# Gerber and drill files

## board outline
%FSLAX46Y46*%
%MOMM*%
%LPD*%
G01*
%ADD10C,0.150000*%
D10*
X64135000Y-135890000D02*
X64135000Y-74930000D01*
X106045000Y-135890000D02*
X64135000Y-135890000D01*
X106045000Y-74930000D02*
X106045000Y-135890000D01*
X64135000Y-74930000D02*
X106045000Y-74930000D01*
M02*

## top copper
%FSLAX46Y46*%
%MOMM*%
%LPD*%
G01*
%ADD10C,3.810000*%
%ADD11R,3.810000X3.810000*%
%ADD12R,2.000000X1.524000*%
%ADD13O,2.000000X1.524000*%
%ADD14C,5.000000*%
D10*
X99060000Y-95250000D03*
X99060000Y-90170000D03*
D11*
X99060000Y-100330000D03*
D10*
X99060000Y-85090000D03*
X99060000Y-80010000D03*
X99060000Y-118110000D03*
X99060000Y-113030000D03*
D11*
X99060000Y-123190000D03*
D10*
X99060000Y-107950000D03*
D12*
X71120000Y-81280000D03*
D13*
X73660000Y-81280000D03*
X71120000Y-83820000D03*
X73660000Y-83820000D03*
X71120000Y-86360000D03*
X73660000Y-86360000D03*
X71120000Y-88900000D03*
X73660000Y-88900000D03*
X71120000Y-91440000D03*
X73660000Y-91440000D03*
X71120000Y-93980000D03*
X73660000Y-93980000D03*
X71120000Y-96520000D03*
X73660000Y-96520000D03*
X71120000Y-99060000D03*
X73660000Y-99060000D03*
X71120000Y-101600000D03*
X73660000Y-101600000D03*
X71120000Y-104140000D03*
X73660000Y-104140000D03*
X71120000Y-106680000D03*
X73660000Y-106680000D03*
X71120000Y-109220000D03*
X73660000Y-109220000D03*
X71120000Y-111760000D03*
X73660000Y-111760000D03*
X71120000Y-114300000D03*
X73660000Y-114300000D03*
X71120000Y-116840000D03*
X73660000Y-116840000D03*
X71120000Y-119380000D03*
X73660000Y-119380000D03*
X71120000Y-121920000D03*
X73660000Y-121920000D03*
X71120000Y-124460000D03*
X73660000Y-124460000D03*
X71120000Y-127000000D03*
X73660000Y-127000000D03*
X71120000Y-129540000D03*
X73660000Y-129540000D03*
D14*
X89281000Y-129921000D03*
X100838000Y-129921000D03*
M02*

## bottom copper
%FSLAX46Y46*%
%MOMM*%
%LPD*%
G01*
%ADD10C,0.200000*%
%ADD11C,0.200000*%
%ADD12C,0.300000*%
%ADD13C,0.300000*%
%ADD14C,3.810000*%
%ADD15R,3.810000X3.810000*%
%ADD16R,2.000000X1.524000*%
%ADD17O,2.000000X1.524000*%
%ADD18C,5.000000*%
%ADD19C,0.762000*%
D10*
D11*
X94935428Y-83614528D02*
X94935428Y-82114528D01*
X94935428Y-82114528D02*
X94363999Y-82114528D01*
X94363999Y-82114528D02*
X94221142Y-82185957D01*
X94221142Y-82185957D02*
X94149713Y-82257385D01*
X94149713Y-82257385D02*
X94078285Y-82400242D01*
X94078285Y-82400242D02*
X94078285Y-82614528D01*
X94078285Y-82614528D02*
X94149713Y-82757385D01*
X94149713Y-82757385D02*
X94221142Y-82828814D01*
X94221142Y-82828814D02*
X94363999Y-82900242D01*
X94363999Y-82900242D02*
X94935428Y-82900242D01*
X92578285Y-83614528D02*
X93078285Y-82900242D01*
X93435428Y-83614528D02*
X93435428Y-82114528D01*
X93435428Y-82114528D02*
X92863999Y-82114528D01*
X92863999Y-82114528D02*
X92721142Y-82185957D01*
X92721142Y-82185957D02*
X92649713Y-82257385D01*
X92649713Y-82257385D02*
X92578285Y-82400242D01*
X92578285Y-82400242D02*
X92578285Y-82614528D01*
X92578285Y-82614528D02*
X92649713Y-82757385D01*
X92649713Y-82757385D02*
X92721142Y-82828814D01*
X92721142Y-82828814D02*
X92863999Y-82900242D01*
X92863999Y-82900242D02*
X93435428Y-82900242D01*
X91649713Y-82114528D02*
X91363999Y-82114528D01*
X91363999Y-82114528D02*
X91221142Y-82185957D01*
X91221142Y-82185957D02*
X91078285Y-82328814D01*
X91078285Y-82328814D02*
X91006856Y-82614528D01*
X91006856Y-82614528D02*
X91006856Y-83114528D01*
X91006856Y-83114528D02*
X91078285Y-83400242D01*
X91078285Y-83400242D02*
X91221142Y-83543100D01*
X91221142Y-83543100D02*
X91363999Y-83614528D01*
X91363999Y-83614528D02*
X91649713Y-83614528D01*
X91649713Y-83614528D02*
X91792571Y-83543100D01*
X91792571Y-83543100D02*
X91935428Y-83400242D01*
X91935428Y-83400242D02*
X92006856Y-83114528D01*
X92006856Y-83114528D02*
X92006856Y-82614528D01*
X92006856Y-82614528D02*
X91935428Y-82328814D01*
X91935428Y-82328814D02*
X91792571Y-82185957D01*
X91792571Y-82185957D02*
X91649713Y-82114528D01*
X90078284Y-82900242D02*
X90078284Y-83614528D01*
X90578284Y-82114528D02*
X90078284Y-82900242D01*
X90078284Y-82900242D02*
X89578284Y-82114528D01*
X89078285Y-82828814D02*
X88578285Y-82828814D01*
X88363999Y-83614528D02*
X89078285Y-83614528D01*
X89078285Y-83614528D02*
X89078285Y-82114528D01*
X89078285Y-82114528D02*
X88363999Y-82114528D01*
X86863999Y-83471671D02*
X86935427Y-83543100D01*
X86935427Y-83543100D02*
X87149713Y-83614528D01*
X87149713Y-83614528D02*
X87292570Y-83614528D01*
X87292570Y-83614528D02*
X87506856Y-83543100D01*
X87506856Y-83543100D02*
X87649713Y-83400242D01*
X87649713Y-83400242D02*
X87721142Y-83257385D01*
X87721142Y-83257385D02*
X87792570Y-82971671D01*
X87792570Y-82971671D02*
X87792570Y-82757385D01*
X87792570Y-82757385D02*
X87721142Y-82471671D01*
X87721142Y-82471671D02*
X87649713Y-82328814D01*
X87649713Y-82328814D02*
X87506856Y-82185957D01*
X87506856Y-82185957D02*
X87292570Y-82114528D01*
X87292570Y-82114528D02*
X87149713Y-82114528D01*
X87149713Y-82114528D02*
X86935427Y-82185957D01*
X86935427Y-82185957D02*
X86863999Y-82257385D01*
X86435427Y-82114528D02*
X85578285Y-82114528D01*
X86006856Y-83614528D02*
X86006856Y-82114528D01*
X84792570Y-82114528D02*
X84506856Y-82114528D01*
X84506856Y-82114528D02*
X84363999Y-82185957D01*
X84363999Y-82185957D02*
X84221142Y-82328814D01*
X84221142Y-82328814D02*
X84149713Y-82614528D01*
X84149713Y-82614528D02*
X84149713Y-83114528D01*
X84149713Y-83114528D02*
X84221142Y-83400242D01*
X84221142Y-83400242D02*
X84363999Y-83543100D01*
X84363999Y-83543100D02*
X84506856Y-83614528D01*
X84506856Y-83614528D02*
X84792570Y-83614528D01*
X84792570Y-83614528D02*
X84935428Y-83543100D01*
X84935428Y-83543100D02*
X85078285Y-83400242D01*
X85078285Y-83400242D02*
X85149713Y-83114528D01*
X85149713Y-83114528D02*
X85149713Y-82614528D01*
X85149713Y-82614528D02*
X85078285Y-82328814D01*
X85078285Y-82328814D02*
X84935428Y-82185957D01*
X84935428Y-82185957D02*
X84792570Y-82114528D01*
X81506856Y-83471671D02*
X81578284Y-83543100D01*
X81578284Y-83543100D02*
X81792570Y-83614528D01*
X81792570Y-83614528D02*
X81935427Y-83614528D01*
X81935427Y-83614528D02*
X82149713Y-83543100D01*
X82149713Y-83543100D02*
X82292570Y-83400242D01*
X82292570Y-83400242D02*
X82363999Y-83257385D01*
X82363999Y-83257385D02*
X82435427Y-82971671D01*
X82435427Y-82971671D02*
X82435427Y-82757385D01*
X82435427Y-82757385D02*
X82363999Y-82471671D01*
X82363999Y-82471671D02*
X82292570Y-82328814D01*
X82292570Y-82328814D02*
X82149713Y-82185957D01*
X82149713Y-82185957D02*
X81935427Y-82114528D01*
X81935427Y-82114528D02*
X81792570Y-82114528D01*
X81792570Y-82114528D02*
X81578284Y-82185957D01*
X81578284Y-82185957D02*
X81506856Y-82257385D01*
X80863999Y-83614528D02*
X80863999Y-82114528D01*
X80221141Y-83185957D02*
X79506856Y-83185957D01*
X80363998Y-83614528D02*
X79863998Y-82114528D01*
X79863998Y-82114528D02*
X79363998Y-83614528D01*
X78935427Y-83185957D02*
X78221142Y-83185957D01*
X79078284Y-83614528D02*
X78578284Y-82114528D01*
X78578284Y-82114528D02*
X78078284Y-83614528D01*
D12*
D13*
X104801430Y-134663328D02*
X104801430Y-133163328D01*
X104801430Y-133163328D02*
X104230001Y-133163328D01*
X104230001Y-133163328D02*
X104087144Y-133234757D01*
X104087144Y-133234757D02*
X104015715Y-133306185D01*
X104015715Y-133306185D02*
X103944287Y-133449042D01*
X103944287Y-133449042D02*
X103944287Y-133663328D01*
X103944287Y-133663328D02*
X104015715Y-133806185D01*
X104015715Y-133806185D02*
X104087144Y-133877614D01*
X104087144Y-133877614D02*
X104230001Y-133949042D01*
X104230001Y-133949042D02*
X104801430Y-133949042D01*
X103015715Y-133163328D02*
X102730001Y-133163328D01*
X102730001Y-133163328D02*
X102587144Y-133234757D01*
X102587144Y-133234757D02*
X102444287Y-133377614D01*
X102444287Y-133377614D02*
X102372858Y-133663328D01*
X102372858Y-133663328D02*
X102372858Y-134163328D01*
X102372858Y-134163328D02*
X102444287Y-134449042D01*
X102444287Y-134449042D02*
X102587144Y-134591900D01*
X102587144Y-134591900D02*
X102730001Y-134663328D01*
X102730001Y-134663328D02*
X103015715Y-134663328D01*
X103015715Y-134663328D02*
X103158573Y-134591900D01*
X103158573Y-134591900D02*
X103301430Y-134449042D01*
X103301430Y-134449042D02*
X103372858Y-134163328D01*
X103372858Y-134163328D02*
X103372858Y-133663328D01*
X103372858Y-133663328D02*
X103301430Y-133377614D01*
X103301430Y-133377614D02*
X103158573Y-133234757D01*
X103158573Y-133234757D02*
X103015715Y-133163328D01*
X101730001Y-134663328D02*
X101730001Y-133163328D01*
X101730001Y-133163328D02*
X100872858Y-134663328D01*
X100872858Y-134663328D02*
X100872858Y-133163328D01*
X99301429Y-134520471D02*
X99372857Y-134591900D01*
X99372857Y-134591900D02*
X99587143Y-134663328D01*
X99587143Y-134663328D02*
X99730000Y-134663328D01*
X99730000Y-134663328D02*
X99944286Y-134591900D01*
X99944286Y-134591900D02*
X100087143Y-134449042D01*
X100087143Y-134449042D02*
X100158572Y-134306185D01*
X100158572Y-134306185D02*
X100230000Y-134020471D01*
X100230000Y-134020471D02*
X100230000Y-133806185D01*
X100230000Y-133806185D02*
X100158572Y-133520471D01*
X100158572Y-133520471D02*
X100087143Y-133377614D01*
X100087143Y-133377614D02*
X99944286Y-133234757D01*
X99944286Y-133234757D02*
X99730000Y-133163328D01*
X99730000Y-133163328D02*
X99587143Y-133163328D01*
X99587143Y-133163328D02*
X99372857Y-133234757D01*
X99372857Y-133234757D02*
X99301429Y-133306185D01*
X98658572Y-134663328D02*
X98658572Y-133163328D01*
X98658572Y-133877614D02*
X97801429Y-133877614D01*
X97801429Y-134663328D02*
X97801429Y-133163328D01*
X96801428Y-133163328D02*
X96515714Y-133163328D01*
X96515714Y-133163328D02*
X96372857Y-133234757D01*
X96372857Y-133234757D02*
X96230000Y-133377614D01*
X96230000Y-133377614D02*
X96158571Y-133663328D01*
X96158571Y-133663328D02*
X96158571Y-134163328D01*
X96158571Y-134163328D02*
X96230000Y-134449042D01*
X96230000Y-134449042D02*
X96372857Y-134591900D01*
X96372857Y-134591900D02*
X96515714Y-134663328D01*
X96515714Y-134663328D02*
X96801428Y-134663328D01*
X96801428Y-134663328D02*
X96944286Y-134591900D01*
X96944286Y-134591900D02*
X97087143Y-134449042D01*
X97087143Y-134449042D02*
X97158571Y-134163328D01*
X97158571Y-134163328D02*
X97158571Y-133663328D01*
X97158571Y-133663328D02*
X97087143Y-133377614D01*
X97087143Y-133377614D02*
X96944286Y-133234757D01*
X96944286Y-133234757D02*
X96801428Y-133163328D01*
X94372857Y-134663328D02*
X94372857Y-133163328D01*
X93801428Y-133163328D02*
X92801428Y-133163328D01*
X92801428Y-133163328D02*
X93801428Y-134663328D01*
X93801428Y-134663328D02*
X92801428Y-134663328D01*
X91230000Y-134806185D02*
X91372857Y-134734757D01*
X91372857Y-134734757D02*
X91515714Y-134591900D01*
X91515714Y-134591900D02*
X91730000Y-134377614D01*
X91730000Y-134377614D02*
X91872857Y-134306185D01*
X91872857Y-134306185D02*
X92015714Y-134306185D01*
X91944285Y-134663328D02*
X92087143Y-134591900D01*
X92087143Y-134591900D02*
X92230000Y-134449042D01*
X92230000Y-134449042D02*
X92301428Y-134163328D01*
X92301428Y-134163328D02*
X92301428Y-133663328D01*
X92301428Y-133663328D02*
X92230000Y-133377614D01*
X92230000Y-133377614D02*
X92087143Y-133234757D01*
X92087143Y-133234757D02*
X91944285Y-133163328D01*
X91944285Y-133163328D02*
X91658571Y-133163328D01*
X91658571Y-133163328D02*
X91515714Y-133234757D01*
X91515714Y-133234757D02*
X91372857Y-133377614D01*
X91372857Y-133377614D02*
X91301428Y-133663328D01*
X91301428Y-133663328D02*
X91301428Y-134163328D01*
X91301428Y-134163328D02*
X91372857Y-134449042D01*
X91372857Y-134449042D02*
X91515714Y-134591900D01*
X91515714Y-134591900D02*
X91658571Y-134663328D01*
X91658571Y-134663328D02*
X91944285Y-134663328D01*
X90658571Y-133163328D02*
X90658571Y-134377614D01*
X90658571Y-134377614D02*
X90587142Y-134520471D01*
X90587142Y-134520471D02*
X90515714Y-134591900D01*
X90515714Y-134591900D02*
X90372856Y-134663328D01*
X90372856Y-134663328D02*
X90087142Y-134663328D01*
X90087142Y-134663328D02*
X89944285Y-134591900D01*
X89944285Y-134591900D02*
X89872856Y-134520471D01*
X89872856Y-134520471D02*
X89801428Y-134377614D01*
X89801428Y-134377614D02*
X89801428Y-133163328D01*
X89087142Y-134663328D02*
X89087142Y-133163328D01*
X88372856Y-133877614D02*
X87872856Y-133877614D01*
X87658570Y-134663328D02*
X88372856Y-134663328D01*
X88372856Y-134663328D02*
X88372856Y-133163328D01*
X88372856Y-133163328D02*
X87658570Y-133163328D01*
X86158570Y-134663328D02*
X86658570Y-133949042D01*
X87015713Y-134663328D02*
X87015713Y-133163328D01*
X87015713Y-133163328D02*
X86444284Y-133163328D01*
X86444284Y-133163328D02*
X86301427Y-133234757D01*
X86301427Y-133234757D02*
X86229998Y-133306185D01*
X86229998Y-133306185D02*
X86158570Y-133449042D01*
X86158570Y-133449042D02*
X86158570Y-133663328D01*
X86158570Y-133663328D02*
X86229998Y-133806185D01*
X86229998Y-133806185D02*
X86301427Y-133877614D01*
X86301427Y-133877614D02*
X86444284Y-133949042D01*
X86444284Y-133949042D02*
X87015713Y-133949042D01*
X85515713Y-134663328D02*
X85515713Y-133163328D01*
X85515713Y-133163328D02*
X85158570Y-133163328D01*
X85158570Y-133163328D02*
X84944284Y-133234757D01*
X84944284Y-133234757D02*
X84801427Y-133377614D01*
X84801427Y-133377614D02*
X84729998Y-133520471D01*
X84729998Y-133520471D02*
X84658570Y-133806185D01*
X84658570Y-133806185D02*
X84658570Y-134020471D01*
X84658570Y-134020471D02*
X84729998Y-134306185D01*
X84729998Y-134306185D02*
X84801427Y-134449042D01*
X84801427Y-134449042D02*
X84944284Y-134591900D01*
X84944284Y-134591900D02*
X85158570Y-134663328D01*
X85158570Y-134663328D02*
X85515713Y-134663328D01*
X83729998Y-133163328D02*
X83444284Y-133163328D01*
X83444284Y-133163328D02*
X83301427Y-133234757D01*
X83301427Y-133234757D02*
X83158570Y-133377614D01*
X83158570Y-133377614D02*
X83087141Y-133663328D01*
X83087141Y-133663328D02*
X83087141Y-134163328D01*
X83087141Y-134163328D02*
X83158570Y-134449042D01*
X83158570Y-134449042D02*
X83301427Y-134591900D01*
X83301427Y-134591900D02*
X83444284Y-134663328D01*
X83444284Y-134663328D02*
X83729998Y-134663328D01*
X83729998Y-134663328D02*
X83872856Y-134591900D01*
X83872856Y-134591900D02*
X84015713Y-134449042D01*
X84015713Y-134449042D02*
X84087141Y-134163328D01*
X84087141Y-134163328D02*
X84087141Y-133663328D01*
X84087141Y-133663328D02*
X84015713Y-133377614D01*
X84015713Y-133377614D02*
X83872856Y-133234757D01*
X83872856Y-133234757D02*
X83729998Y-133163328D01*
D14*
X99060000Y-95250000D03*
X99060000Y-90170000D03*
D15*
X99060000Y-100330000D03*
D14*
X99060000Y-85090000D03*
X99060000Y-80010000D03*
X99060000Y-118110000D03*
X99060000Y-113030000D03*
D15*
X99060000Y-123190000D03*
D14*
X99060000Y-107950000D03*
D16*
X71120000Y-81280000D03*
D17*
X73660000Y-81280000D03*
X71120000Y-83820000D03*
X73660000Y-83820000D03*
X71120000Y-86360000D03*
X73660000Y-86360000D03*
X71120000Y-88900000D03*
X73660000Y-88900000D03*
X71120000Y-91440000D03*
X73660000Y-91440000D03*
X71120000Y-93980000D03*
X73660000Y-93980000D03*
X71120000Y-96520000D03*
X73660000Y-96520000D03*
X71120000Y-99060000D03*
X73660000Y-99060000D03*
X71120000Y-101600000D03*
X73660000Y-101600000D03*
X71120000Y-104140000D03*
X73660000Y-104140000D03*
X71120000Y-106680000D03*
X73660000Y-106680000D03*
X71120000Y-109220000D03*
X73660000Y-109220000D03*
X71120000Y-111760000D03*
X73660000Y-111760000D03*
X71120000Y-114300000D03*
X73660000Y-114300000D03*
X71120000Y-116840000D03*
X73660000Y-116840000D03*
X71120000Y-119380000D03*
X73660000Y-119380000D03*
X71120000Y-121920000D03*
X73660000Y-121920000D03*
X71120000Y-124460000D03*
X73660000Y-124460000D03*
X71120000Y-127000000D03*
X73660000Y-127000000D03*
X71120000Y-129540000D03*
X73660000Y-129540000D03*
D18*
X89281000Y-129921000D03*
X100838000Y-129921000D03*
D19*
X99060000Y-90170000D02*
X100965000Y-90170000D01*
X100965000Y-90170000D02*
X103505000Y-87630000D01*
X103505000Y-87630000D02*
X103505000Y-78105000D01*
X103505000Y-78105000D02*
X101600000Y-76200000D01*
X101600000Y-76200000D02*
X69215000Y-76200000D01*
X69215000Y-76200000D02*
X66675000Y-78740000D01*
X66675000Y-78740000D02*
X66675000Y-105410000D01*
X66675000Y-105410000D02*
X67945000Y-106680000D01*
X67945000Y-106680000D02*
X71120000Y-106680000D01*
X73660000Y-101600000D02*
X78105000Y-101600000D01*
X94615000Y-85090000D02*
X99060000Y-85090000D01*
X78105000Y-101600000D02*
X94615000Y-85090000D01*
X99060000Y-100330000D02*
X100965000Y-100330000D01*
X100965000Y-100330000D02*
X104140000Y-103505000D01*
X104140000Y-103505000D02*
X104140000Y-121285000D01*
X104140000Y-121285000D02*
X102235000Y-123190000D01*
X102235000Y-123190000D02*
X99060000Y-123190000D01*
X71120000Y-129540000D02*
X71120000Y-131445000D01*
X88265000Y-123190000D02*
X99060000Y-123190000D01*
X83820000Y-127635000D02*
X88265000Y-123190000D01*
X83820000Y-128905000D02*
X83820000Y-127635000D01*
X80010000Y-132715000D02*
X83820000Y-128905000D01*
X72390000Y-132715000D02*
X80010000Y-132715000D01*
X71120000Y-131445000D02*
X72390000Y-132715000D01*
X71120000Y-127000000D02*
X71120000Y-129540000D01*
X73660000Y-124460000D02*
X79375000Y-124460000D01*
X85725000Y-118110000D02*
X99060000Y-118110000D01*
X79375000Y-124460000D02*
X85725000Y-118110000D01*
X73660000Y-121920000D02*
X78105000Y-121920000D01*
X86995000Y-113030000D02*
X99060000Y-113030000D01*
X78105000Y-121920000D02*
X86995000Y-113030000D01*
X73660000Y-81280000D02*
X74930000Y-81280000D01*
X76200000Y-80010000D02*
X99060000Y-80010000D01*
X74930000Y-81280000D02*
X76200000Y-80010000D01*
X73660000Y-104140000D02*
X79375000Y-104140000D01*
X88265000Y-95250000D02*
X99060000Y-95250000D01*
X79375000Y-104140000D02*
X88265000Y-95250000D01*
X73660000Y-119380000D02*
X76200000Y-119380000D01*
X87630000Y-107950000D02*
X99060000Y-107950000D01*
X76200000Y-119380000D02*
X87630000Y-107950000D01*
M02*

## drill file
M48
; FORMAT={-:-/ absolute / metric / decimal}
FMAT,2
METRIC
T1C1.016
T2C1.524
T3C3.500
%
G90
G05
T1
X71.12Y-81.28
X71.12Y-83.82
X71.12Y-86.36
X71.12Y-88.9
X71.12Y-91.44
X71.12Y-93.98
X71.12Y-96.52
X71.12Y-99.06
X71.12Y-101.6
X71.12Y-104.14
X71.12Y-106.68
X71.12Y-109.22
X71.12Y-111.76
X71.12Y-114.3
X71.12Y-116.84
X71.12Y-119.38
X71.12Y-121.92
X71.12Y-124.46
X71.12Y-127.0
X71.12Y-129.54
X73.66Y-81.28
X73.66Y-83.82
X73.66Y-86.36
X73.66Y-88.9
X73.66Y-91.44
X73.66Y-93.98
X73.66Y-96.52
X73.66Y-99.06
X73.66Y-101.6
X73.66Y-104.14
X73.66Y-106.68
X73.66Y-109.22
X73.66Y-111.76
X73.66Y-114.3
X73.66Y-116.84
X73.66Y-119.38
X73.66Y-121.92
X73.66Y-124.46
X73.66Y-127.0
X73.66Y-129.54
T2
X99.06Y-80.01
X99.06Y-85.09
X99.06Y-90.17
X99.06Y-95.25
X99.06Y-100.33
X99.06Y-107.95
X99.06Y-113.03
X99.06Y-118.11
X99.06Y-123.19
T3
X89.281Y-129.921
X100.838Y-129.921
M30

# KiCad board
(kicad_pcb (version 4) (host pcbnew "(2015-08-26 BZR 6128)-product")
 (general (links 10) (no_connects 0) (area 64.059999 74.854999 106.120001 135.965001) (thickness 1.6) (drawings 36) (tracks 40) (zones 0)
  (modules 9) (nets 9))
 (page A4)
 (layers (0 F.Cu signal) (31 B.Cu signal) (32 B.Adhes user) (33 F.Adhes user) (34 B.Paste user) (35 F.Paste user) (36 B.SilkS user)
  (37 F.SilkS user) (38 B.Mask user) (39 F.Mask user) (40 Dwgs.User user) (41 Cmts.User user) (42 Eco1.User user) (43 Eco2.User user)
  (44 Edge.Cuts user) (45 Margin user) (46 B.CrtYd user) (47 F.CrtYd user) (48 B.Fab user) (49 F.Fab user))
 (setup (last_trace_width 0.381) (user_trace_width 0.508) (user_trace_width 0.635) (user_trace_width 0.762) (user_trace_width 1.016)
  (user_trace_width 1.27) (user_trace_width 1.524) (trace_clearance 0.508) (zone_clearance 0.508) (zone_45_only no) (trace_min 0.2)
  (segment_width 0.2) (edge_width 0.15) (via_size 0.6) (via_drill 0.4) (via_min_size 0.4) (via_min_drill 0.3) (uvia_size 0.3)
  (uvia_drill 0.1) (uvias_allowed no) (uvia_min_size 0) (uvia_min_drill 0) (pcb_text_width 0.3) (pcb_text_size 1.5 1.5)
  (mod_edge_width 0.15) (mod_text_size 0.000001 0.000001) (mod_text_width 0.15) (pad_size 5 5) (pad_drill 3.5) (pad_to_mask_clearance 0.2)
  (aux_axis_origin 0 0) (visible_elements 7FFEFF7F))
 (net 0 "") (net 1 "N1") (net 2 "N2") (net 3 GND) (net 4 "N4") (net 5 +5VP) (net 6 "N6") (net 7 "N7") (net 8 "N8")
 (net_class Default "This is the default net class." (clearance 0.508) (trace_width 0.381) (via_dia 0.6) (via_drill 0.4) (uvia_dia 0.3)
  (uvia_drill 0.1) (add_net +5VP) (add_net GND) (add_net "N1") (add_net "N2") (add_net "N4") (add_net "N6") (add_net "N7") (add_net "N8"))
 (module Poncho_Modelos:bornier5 (layer F.Cu) (at 99.06 90.17 90)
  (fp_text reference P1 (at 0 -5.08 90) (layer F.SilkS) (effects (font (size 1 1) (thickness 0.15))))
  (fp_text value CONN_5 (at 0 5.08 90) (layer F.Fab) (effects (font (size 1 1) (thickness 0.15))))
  (pad 2 thru_hole circle (at -5.08 0 90) (size 3.81 3.81) (drill 1.524) (layers *.Cu *.Mask F.SilkS) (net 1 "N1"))
  (pad 3 thru_hole circle (at 0 0 90) (size 3.81 3.81) (drill 1.524) (layers *.Cu *.Mask F.SilkS) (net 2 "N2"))
  (pad 1 thru_hole rect (at -10.16 0 90) (size 3.81 3.81) (drill 1.524) (layers *.Cu *.Mask F.SilkS) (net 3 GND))
  (pad 4 thru_hole circle (at 5.08 0 90) (size 3.81 3.81) (drill 1.524) (layers *.Cu *.Mask F.SilkS) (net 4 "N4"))
  (pad 5 thru_hole circle (at 10.16 0 90) (size 3.81 3.81) (drill 1.524) (layers *.Cu *.Mask F.SilkS) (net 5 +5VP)))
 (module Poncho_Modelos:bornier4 (layer F.Cu) (at 99.06 115.57 90)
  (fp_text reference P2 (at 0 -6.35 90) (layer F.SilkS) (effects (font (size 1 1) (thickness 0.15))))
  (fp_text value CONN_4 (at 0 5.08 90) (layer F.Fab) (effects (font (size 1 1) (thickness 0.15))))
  (pad 2 thru_hole circle (at -2.54 0 90) (size 3.81 3.81) (drill 1.524) (layers *.Cu *.Mask F.SilkS) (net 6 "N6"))
  (pad 3 thru_hole circle (at 2.54 0 90) (size 3.81 3.81) (drill 1.524) (layers *.Cu *.Mask F.SilkS) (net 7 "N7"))
  (pad 1 thru_hole rect (at -7.62 0 90) (size 3.81 3.81) (drill 1.524) (layers *.Cu *.Mask F.SilkS) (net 3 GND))
  (pad 4 thru_hole circle (at 7.62 0 90) (size 3.81 3.81) (drill 1.524) (layers *.Cu *.Mask F.SilkS) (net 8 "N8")))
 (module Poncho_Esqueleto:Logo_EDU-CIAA (layer F.Cu) (at 89.535 116.205)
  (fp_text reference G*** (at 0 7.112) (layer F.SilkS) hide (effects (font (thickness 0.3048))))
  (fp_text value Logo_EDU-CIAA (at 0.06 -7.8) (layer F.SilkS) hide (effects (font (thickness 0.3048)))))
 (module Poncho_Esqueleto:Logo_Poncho (layer F.Cu) (at 88.265 91.44)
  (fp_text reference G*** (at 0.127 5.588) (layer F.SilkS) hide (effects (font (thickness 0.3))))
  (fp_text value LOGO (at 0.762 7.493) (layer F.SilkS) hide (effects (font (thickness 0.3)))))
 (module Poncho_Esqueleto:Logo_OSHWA (layer F.Cu) (at 88.9 101.6)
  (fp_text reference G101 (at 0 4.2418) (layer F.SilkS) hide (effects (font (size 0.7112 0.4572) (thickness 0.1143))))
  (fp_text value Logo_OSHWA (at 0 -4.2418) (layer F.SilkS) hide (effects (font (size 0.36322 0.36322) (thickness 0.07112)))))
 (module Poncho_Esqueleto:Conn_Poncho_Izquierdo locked (layer F.Cu) (at 71.12 81.28)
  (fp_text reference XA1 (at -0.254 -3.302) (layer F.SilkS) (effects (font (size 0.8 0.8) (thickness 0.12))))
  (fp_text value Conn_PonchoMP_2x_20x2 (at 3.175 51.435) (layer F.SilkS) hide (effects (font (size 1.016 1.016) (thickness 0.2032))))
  (pad 41 thru_hole rect (at 0 0 270) (size 1.524 2) (drill 1.016) (layers *.Cu *.Mask F.SilkS))
  (pad 42 thru_hole oval (at 2.54 0 270) (size 1.524 2) (drill 1.016) (layers *.Cu *.Mask F.SilkS) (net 5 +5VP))
  (pad 43 thru_hole oval (at 0 2.54 270) (size 1.524 2) (drill 1.016) (layers *.Cu *.Mask F.SilkS))
  (pad 44 thru_hole oval (at 2.54 2.54 270) (size 1.524 2) (drill 1.016) (layers *.Cu *.Mask F.SilkS))
  (pad 45 thru_hole oval (at 0 5.08 270) (size 1.524 2) (drill 1.016) (layers *.Cu *.Mask F.SilkS))
  (pad 46 thru_hole oval (at 2.54 5.08 270) (size 1.524 2) (drill 1.016) (layers *.Cu *.Mask F.SilkS))
  (pad 47 thru_hole oval (at 0 7.62 270) (size 1.524 2) (drill 1.016) (layers *.Cu *.Mask F.SilkS))
  (pad 48 thru_hole oval (at 2.54 7.62 270) (size 1.524 2) (drill 1.016) (layers *.Cu *.Mask F.SilkS))
  (pad 49 thru_hole oval (at 0 10.16 270) (size 1.524 2) (drill 1.016) (layers *.Cu *.Mask F.SilkS))
  (pad 50 thru_hole oval (at 2.54 10.16 270) (size 1.524 2) (drill 1.016) (layers *.Cu *.Mask F.SilkS))
  (pad 51 thru_hole oval (at 0 12.7 270) (size 1.524 2) (drill 1.016) (layers *.Cu *.Mask F.SilkS))
  (pad 52 thru_hole oval (at 2.54 12.7 270) (size 1.524 2) (drill 1.016) (layers *.Cu *.Mask F.SilkS))
  (pad 53 thru_hole oval (at 0 15.24 270) (size 1.524 2) (drill 1.016) (layers *.Cu *.Mask F.SilkS))
  (pad 54 thru_hole oval (at 2.54 15.24 270) (size 1.524 2) (drill 1.016) (layers *.Cu *.Mask F.SilkS))
  (pad 55 thru_hole oval (at 0 17.78 270) (size 1.524 2) (drill 1.016) (layers *.Cu *.Mask F.SilkS))
  (pad 56 thru_hole oval (at 2.54 17.78 270) (size 1.524 2) (drill 1.016) (layers *.Cu *.Mask F.SilkS))
  (pad 57 thru_hole oval (at 0 20.32 270) (size 1.524 2) (drill 1.016) (layers *.Cu *.Mask F.SilkS))
  (pad 58 thru_hole oval (at 2.54 20.32 270) (size 1.524 2) (drill 1.016) (layers *.Cu *.Mask F.SilkS) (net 4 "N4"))
  (pad 59 thru_hole oval (at 0 22.86 270) (size 1.524 2) (drill 1.016) (layers *.Cu *.Mask F.SilkS))
  (pad 60 thru_hole oval (at 2.54 22.86 270) (size 1.524 2) (drill 1.016) (layers *.Cu *.Mask F.SilkS) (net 1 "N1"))
  (pad 61 thru_hole oval (at 0 25.4 270) (size 1.524 2) (drill 1.016) (layers *.Cu *.Mask F.SilkS) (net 2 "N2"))
  (pad 62 thru_hole oval (at 2.54 25.4 270) (size 1.524 2) (drill 1.016) (layers *.Cu *.Mask F.SilkS))
  (pad 63 thru_hole oval (at 0 27.94 270) (size 1.524 2) (drill 1.016) (layers *.Cu *.Mask F.SilkS))
  (pad 64 thru_hole oval (at 2.54 27.94 270) (size 1.524 2) (drill 1.016) (layers *.Cu *.Mask F.SilkS))
  (pad 65 thru_hole oval (at 0 30.48 270) (size 1.524 2) (drill 1.016) (layers *.Cu *.Mask F.SilkS))
  (pad 66 thru_hole oval (at 2.54 30.48 270) (size 1.524 2) (drill 1.016) (layers *.Cu *.Mask F.SilkS))
  (pad 67 thru_hole oval (at 0 33.02 270) (size 1.524 2) (drill 1.016) (layers *.Cu *.Mask F.SilkS))
  (pad 68 thru_hole oval (at 2.54 33.02 270) (size 1.524 2) (drill 1.016) (layers *.Cu *.Mask F.SilkS))
  (pad 69 thru_hole oval (at 0 35.56 270) (size 1.524 2) (drill 1.016) (layers *.Cu *.Mask F.SilkS))
  (pad 70 thru_hole oval (at 2.54 35.56 270) (size 1.524 2) (drill 1.016) (layers *.Cu *.Mask F.SilkS))
  (pad 71 thru_hole oval (at 0 38.1 270) (size 1.524 2) (drill 1.016) (layers *.Cu *.Mask F.SilkS))
  (pad 72 thru_hole oval (at 2.54 38.1 270) (size 1.524 2) (drill 1.016) (layers *.Cu *.Mask F.SilkS) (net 8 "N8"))
  (pad 73 thru_hole oval (at 0 40.64 270) (size 1.524 2) (drill 1.016) (layers *.Cu *.Mask F.SilkS))
  (pad 74 thru_hole oval (at 2.54 40.64 270) (size 1.524 2) (drill 1.016) (layers *.Cu *.Mask F.SilkS) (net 7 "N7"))
  (pad 75 thru_hole oval (at 0 43.18 270) (size 1.524 2) (drill 1.016) (layers *.Cu *.Mask F.SilkS))
  (pad 76 thru_hole oval (at 2.54 43.18 270) (size 1.524 2) (drill 1.016) (layers *.Cu *.Mask F.SilkS) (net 6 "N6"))
  (pad 77 thru_hole oval (at 0 45.72 270) (size 1.524 2) (drill 1.016) (layers *.Cu *.Mask F.SilkS) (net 3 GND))
  (pad 78 thru_hole oval (at 2.54 45.72 270) (size 1.524 2) (drill 1.016) (layers *.Cu *.Mask F.SilkS))
  (pad 79 thru_hole oval (at 0 48.26 270) (size 1.524 2) (drill 1.016) (layers *.Cu *.Mask F.SilkS) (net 3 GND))
  (pad 80 thru_hole oval (at 2.54 48.26 270) (size 1.524 2) (drill 1.016) (layers *.Cu *.Mask F.SilkS)))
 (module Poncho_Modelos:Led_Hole (layer F.Cu) (at 89.281 129.921)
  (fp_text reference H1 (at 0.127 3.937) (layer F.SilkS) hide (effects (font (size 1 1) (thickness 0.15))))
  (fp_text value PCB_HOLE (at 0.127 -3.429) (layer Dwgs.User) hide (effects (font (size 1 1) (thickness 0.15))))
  (pad 1 thru_hole circle (at 0 0) (size 5 5) (drill 3.5) (layers *.Cu *.Mask F.SilkS)))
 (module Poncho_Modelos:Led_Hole (layer F.Cu) (at 100.838 129.921)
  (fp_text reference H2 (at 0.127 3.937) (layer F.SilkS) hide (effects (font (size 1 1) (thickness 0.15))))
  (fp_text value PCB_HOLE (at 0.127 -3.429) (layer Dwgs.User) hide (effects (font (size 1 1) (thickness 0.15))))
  (pad 1 thru_hole circle (at 0 0) (size 5 5) (drill 3.5) (layers *.Cu *.Mask F.SilkS)))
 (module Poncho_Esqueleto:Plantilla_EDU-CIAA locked (layer F.Cu) (at 142.24 81.28)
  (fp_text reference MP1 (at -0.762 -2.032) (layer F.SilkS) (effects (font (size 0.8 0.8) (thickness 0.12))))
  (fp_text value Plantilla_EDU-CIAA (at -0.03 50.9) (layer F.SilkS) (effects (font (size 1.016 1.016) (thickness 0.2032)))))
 (gr_line (start 64.135 135.89) (end 64.135 74.93) (angle 90) (layer Edge.Cuts) (width 0.15))
 (gr_line (start 106.045 135.89) (end 64.135 135.89) (angle 90) (layer Edge.Cuts) (width 0.15))
 (gr_line (start 106.045 74.93) (end 106.045 135.89) (angle 90) (layer Edge.Cuts) (width 0.15))
 (gr_line (start 64.135 74.93) (end 106.045 74.93) (angle 90) (layer Edge.Cuts) (width 0.15))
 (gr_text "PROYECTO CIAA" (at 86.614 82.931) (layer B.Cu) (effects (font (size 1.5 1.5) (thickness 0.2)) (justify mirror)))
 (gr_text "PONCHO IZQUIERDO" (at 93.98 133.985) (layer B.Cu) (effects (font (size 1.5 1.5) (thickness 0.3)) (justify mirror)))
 (segment (start 99.06 90.17) (end 100.965 90.17) (width 0.762) (layer B.Cu) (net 2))
 (segment (start 100.965 90.17) (end 103.505 87.63) (width 0.762) (layer B.Cu) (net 2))
 (segment (start 103.505 87.63) (end 103.505 78.105) (width 0.762) (layer B.Cu) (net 2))
 (segment (start 103.505 78.105) (end 101.6 76.2) (width 0.762) (layer B.Cu) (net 2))
 (segment (start 101.6 76.2) (end 69.215 76.2) (width 0.762) (layer B.Cu) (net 2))
 (segment (start 69.215 76.2) (end 66.675 78.74) (width 0.762) (layer B.Cu) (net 2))
 (segment (start 66.675 78.74) (end 66.675 105.41) (width 0.762) (layer B.Cu) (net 2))
 (segment (start 66.675 105.41) (end 67.945 106.68) (width 0.762) (layer B.Cu) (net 2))
 (segment (start 67.945 106.68) (end 71.12 106.68) (width 0.762) (layer B.Cu) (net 2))
 (segment (start 73.66 101.6) (end 78.105 101.6) (width 0.762) (layer B.Cu) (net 4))
 (segment (start 94.615 85.09) (end 99.06 85.09) (width 0.762) (layer B.Cu) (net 4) (status 20))
 (segment (start 78.105 101.6) (end 94.615 85.09) (width 0.762) (layer B.Cu) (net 4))
 (segment (start 99.06 100.33) (end 100.965 100.33) (width 0.762) (layer B.Cu) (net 3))
 (segment (start 100.965 100.33) (end 104.14 103.505) (width 0.762) (layer B.Cu) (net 3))
 (segment (start 104.14 103.505) (end 104.14 121.285) (width 0.762) (layer B.Cu) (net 3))
 (segment (start 104.14 121.285) (end 102.235 123.19) (width 0.762) (layer B.Cu) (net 3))
 (segment (start 102.235 123.19) (end 99.06 123.19) (width 0.762) (layer B.Cu) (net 3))
 (segment (start 71.12 129.54) (end 71.12 131.445) (width 0.762) (layer B.Cu) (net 3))
 (segment (start 88.265 123.19) (end 99.06 123.19) (width 0.762) (layer B.Cu) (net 3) (status 20))
 (segment (start 83.82 127.635) (end 88.265 123.19) (width 0.762) (layer B.Cu) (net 3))
 (segment (start 83.82 128.905) (end 83.82 127.635) (width 0.762) (layer B.Cu) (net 3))
 (segment (start 80.01 132.715) (end 83.82 128.905) (width 0.762) (layer B.Cu) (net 3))
 (segment (start 72.39 132.715) (end 80.01 132.715) (width 0.762) (layer B.Cu) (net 3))
 (segment (start 71.12 131.445) (end 72.39 132.715) (width 0.762) (layer B.Cu) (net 3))
 (segment (start 71.12 127) (end 71.12 129.54) (width 0.762) (layer B.Cu) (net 3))
 (segment (start 73.66 124.46) (end 79.375 124.46) (width 0.762) (layer B.Cu) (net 6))
 (segment (start 85.725 118.11) (end 99.06 118.11) (width 0.762) (layer B.Cu) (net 6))
 (segment (start 79.375 124.46) (end 85.725 118.11) (width 0.762) (layer B.Cu) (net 6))
 (segment (start 73.66 121.92) (end 78.105 121.92) (width 0.762) (layer B.Cu) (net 7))
 (segment (start 86.995 113.03) (end 99.06 113.03) (width 0.762) (layer B.Cu) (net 7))
 (segment (start 78.105 121.92) (end 86.995 113.03) (width 0.762) (layer B.Cu) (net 7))
 (segment (start 73.66 81.28) (end 74.93 81.28) (width 0.762) (layer B.Cu) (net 5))
 (segment (start 76.2 80.01) (end 99.06 80.01) (width 0.762) (layer B.Cu) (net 5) (status 20))
 (segment (start 74.93 81.28) (end 76.2 80.01) (width 0.762) (layer B.Cu) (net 5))
 (segment (start 73.66 104.14) (end 79.375 104.14) (width 0.762) (layer B.Cu) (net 1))
 (segment (start 88.265 95.25) (end 99.06 95.25) (width 0.762) (layer B.Cu) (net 1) (status 20))
 (segment (start 79.375 104.14) (end 88.265 95.25) (width 0.762) (layer B.Cu) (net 1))
 (segment (start 73.66 119.38) (end 76.2 119.38) (width 0.762) (layer B.Cu) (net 8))
 (segment (start 87.63 107.95) (end 99.06 107.95) (width 0.762) (layer B.Cu) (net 8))
 (segment (start 76.2 119.38) (end 87.63 107.95) (width 0.762) (layer B.Cu) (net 8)))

